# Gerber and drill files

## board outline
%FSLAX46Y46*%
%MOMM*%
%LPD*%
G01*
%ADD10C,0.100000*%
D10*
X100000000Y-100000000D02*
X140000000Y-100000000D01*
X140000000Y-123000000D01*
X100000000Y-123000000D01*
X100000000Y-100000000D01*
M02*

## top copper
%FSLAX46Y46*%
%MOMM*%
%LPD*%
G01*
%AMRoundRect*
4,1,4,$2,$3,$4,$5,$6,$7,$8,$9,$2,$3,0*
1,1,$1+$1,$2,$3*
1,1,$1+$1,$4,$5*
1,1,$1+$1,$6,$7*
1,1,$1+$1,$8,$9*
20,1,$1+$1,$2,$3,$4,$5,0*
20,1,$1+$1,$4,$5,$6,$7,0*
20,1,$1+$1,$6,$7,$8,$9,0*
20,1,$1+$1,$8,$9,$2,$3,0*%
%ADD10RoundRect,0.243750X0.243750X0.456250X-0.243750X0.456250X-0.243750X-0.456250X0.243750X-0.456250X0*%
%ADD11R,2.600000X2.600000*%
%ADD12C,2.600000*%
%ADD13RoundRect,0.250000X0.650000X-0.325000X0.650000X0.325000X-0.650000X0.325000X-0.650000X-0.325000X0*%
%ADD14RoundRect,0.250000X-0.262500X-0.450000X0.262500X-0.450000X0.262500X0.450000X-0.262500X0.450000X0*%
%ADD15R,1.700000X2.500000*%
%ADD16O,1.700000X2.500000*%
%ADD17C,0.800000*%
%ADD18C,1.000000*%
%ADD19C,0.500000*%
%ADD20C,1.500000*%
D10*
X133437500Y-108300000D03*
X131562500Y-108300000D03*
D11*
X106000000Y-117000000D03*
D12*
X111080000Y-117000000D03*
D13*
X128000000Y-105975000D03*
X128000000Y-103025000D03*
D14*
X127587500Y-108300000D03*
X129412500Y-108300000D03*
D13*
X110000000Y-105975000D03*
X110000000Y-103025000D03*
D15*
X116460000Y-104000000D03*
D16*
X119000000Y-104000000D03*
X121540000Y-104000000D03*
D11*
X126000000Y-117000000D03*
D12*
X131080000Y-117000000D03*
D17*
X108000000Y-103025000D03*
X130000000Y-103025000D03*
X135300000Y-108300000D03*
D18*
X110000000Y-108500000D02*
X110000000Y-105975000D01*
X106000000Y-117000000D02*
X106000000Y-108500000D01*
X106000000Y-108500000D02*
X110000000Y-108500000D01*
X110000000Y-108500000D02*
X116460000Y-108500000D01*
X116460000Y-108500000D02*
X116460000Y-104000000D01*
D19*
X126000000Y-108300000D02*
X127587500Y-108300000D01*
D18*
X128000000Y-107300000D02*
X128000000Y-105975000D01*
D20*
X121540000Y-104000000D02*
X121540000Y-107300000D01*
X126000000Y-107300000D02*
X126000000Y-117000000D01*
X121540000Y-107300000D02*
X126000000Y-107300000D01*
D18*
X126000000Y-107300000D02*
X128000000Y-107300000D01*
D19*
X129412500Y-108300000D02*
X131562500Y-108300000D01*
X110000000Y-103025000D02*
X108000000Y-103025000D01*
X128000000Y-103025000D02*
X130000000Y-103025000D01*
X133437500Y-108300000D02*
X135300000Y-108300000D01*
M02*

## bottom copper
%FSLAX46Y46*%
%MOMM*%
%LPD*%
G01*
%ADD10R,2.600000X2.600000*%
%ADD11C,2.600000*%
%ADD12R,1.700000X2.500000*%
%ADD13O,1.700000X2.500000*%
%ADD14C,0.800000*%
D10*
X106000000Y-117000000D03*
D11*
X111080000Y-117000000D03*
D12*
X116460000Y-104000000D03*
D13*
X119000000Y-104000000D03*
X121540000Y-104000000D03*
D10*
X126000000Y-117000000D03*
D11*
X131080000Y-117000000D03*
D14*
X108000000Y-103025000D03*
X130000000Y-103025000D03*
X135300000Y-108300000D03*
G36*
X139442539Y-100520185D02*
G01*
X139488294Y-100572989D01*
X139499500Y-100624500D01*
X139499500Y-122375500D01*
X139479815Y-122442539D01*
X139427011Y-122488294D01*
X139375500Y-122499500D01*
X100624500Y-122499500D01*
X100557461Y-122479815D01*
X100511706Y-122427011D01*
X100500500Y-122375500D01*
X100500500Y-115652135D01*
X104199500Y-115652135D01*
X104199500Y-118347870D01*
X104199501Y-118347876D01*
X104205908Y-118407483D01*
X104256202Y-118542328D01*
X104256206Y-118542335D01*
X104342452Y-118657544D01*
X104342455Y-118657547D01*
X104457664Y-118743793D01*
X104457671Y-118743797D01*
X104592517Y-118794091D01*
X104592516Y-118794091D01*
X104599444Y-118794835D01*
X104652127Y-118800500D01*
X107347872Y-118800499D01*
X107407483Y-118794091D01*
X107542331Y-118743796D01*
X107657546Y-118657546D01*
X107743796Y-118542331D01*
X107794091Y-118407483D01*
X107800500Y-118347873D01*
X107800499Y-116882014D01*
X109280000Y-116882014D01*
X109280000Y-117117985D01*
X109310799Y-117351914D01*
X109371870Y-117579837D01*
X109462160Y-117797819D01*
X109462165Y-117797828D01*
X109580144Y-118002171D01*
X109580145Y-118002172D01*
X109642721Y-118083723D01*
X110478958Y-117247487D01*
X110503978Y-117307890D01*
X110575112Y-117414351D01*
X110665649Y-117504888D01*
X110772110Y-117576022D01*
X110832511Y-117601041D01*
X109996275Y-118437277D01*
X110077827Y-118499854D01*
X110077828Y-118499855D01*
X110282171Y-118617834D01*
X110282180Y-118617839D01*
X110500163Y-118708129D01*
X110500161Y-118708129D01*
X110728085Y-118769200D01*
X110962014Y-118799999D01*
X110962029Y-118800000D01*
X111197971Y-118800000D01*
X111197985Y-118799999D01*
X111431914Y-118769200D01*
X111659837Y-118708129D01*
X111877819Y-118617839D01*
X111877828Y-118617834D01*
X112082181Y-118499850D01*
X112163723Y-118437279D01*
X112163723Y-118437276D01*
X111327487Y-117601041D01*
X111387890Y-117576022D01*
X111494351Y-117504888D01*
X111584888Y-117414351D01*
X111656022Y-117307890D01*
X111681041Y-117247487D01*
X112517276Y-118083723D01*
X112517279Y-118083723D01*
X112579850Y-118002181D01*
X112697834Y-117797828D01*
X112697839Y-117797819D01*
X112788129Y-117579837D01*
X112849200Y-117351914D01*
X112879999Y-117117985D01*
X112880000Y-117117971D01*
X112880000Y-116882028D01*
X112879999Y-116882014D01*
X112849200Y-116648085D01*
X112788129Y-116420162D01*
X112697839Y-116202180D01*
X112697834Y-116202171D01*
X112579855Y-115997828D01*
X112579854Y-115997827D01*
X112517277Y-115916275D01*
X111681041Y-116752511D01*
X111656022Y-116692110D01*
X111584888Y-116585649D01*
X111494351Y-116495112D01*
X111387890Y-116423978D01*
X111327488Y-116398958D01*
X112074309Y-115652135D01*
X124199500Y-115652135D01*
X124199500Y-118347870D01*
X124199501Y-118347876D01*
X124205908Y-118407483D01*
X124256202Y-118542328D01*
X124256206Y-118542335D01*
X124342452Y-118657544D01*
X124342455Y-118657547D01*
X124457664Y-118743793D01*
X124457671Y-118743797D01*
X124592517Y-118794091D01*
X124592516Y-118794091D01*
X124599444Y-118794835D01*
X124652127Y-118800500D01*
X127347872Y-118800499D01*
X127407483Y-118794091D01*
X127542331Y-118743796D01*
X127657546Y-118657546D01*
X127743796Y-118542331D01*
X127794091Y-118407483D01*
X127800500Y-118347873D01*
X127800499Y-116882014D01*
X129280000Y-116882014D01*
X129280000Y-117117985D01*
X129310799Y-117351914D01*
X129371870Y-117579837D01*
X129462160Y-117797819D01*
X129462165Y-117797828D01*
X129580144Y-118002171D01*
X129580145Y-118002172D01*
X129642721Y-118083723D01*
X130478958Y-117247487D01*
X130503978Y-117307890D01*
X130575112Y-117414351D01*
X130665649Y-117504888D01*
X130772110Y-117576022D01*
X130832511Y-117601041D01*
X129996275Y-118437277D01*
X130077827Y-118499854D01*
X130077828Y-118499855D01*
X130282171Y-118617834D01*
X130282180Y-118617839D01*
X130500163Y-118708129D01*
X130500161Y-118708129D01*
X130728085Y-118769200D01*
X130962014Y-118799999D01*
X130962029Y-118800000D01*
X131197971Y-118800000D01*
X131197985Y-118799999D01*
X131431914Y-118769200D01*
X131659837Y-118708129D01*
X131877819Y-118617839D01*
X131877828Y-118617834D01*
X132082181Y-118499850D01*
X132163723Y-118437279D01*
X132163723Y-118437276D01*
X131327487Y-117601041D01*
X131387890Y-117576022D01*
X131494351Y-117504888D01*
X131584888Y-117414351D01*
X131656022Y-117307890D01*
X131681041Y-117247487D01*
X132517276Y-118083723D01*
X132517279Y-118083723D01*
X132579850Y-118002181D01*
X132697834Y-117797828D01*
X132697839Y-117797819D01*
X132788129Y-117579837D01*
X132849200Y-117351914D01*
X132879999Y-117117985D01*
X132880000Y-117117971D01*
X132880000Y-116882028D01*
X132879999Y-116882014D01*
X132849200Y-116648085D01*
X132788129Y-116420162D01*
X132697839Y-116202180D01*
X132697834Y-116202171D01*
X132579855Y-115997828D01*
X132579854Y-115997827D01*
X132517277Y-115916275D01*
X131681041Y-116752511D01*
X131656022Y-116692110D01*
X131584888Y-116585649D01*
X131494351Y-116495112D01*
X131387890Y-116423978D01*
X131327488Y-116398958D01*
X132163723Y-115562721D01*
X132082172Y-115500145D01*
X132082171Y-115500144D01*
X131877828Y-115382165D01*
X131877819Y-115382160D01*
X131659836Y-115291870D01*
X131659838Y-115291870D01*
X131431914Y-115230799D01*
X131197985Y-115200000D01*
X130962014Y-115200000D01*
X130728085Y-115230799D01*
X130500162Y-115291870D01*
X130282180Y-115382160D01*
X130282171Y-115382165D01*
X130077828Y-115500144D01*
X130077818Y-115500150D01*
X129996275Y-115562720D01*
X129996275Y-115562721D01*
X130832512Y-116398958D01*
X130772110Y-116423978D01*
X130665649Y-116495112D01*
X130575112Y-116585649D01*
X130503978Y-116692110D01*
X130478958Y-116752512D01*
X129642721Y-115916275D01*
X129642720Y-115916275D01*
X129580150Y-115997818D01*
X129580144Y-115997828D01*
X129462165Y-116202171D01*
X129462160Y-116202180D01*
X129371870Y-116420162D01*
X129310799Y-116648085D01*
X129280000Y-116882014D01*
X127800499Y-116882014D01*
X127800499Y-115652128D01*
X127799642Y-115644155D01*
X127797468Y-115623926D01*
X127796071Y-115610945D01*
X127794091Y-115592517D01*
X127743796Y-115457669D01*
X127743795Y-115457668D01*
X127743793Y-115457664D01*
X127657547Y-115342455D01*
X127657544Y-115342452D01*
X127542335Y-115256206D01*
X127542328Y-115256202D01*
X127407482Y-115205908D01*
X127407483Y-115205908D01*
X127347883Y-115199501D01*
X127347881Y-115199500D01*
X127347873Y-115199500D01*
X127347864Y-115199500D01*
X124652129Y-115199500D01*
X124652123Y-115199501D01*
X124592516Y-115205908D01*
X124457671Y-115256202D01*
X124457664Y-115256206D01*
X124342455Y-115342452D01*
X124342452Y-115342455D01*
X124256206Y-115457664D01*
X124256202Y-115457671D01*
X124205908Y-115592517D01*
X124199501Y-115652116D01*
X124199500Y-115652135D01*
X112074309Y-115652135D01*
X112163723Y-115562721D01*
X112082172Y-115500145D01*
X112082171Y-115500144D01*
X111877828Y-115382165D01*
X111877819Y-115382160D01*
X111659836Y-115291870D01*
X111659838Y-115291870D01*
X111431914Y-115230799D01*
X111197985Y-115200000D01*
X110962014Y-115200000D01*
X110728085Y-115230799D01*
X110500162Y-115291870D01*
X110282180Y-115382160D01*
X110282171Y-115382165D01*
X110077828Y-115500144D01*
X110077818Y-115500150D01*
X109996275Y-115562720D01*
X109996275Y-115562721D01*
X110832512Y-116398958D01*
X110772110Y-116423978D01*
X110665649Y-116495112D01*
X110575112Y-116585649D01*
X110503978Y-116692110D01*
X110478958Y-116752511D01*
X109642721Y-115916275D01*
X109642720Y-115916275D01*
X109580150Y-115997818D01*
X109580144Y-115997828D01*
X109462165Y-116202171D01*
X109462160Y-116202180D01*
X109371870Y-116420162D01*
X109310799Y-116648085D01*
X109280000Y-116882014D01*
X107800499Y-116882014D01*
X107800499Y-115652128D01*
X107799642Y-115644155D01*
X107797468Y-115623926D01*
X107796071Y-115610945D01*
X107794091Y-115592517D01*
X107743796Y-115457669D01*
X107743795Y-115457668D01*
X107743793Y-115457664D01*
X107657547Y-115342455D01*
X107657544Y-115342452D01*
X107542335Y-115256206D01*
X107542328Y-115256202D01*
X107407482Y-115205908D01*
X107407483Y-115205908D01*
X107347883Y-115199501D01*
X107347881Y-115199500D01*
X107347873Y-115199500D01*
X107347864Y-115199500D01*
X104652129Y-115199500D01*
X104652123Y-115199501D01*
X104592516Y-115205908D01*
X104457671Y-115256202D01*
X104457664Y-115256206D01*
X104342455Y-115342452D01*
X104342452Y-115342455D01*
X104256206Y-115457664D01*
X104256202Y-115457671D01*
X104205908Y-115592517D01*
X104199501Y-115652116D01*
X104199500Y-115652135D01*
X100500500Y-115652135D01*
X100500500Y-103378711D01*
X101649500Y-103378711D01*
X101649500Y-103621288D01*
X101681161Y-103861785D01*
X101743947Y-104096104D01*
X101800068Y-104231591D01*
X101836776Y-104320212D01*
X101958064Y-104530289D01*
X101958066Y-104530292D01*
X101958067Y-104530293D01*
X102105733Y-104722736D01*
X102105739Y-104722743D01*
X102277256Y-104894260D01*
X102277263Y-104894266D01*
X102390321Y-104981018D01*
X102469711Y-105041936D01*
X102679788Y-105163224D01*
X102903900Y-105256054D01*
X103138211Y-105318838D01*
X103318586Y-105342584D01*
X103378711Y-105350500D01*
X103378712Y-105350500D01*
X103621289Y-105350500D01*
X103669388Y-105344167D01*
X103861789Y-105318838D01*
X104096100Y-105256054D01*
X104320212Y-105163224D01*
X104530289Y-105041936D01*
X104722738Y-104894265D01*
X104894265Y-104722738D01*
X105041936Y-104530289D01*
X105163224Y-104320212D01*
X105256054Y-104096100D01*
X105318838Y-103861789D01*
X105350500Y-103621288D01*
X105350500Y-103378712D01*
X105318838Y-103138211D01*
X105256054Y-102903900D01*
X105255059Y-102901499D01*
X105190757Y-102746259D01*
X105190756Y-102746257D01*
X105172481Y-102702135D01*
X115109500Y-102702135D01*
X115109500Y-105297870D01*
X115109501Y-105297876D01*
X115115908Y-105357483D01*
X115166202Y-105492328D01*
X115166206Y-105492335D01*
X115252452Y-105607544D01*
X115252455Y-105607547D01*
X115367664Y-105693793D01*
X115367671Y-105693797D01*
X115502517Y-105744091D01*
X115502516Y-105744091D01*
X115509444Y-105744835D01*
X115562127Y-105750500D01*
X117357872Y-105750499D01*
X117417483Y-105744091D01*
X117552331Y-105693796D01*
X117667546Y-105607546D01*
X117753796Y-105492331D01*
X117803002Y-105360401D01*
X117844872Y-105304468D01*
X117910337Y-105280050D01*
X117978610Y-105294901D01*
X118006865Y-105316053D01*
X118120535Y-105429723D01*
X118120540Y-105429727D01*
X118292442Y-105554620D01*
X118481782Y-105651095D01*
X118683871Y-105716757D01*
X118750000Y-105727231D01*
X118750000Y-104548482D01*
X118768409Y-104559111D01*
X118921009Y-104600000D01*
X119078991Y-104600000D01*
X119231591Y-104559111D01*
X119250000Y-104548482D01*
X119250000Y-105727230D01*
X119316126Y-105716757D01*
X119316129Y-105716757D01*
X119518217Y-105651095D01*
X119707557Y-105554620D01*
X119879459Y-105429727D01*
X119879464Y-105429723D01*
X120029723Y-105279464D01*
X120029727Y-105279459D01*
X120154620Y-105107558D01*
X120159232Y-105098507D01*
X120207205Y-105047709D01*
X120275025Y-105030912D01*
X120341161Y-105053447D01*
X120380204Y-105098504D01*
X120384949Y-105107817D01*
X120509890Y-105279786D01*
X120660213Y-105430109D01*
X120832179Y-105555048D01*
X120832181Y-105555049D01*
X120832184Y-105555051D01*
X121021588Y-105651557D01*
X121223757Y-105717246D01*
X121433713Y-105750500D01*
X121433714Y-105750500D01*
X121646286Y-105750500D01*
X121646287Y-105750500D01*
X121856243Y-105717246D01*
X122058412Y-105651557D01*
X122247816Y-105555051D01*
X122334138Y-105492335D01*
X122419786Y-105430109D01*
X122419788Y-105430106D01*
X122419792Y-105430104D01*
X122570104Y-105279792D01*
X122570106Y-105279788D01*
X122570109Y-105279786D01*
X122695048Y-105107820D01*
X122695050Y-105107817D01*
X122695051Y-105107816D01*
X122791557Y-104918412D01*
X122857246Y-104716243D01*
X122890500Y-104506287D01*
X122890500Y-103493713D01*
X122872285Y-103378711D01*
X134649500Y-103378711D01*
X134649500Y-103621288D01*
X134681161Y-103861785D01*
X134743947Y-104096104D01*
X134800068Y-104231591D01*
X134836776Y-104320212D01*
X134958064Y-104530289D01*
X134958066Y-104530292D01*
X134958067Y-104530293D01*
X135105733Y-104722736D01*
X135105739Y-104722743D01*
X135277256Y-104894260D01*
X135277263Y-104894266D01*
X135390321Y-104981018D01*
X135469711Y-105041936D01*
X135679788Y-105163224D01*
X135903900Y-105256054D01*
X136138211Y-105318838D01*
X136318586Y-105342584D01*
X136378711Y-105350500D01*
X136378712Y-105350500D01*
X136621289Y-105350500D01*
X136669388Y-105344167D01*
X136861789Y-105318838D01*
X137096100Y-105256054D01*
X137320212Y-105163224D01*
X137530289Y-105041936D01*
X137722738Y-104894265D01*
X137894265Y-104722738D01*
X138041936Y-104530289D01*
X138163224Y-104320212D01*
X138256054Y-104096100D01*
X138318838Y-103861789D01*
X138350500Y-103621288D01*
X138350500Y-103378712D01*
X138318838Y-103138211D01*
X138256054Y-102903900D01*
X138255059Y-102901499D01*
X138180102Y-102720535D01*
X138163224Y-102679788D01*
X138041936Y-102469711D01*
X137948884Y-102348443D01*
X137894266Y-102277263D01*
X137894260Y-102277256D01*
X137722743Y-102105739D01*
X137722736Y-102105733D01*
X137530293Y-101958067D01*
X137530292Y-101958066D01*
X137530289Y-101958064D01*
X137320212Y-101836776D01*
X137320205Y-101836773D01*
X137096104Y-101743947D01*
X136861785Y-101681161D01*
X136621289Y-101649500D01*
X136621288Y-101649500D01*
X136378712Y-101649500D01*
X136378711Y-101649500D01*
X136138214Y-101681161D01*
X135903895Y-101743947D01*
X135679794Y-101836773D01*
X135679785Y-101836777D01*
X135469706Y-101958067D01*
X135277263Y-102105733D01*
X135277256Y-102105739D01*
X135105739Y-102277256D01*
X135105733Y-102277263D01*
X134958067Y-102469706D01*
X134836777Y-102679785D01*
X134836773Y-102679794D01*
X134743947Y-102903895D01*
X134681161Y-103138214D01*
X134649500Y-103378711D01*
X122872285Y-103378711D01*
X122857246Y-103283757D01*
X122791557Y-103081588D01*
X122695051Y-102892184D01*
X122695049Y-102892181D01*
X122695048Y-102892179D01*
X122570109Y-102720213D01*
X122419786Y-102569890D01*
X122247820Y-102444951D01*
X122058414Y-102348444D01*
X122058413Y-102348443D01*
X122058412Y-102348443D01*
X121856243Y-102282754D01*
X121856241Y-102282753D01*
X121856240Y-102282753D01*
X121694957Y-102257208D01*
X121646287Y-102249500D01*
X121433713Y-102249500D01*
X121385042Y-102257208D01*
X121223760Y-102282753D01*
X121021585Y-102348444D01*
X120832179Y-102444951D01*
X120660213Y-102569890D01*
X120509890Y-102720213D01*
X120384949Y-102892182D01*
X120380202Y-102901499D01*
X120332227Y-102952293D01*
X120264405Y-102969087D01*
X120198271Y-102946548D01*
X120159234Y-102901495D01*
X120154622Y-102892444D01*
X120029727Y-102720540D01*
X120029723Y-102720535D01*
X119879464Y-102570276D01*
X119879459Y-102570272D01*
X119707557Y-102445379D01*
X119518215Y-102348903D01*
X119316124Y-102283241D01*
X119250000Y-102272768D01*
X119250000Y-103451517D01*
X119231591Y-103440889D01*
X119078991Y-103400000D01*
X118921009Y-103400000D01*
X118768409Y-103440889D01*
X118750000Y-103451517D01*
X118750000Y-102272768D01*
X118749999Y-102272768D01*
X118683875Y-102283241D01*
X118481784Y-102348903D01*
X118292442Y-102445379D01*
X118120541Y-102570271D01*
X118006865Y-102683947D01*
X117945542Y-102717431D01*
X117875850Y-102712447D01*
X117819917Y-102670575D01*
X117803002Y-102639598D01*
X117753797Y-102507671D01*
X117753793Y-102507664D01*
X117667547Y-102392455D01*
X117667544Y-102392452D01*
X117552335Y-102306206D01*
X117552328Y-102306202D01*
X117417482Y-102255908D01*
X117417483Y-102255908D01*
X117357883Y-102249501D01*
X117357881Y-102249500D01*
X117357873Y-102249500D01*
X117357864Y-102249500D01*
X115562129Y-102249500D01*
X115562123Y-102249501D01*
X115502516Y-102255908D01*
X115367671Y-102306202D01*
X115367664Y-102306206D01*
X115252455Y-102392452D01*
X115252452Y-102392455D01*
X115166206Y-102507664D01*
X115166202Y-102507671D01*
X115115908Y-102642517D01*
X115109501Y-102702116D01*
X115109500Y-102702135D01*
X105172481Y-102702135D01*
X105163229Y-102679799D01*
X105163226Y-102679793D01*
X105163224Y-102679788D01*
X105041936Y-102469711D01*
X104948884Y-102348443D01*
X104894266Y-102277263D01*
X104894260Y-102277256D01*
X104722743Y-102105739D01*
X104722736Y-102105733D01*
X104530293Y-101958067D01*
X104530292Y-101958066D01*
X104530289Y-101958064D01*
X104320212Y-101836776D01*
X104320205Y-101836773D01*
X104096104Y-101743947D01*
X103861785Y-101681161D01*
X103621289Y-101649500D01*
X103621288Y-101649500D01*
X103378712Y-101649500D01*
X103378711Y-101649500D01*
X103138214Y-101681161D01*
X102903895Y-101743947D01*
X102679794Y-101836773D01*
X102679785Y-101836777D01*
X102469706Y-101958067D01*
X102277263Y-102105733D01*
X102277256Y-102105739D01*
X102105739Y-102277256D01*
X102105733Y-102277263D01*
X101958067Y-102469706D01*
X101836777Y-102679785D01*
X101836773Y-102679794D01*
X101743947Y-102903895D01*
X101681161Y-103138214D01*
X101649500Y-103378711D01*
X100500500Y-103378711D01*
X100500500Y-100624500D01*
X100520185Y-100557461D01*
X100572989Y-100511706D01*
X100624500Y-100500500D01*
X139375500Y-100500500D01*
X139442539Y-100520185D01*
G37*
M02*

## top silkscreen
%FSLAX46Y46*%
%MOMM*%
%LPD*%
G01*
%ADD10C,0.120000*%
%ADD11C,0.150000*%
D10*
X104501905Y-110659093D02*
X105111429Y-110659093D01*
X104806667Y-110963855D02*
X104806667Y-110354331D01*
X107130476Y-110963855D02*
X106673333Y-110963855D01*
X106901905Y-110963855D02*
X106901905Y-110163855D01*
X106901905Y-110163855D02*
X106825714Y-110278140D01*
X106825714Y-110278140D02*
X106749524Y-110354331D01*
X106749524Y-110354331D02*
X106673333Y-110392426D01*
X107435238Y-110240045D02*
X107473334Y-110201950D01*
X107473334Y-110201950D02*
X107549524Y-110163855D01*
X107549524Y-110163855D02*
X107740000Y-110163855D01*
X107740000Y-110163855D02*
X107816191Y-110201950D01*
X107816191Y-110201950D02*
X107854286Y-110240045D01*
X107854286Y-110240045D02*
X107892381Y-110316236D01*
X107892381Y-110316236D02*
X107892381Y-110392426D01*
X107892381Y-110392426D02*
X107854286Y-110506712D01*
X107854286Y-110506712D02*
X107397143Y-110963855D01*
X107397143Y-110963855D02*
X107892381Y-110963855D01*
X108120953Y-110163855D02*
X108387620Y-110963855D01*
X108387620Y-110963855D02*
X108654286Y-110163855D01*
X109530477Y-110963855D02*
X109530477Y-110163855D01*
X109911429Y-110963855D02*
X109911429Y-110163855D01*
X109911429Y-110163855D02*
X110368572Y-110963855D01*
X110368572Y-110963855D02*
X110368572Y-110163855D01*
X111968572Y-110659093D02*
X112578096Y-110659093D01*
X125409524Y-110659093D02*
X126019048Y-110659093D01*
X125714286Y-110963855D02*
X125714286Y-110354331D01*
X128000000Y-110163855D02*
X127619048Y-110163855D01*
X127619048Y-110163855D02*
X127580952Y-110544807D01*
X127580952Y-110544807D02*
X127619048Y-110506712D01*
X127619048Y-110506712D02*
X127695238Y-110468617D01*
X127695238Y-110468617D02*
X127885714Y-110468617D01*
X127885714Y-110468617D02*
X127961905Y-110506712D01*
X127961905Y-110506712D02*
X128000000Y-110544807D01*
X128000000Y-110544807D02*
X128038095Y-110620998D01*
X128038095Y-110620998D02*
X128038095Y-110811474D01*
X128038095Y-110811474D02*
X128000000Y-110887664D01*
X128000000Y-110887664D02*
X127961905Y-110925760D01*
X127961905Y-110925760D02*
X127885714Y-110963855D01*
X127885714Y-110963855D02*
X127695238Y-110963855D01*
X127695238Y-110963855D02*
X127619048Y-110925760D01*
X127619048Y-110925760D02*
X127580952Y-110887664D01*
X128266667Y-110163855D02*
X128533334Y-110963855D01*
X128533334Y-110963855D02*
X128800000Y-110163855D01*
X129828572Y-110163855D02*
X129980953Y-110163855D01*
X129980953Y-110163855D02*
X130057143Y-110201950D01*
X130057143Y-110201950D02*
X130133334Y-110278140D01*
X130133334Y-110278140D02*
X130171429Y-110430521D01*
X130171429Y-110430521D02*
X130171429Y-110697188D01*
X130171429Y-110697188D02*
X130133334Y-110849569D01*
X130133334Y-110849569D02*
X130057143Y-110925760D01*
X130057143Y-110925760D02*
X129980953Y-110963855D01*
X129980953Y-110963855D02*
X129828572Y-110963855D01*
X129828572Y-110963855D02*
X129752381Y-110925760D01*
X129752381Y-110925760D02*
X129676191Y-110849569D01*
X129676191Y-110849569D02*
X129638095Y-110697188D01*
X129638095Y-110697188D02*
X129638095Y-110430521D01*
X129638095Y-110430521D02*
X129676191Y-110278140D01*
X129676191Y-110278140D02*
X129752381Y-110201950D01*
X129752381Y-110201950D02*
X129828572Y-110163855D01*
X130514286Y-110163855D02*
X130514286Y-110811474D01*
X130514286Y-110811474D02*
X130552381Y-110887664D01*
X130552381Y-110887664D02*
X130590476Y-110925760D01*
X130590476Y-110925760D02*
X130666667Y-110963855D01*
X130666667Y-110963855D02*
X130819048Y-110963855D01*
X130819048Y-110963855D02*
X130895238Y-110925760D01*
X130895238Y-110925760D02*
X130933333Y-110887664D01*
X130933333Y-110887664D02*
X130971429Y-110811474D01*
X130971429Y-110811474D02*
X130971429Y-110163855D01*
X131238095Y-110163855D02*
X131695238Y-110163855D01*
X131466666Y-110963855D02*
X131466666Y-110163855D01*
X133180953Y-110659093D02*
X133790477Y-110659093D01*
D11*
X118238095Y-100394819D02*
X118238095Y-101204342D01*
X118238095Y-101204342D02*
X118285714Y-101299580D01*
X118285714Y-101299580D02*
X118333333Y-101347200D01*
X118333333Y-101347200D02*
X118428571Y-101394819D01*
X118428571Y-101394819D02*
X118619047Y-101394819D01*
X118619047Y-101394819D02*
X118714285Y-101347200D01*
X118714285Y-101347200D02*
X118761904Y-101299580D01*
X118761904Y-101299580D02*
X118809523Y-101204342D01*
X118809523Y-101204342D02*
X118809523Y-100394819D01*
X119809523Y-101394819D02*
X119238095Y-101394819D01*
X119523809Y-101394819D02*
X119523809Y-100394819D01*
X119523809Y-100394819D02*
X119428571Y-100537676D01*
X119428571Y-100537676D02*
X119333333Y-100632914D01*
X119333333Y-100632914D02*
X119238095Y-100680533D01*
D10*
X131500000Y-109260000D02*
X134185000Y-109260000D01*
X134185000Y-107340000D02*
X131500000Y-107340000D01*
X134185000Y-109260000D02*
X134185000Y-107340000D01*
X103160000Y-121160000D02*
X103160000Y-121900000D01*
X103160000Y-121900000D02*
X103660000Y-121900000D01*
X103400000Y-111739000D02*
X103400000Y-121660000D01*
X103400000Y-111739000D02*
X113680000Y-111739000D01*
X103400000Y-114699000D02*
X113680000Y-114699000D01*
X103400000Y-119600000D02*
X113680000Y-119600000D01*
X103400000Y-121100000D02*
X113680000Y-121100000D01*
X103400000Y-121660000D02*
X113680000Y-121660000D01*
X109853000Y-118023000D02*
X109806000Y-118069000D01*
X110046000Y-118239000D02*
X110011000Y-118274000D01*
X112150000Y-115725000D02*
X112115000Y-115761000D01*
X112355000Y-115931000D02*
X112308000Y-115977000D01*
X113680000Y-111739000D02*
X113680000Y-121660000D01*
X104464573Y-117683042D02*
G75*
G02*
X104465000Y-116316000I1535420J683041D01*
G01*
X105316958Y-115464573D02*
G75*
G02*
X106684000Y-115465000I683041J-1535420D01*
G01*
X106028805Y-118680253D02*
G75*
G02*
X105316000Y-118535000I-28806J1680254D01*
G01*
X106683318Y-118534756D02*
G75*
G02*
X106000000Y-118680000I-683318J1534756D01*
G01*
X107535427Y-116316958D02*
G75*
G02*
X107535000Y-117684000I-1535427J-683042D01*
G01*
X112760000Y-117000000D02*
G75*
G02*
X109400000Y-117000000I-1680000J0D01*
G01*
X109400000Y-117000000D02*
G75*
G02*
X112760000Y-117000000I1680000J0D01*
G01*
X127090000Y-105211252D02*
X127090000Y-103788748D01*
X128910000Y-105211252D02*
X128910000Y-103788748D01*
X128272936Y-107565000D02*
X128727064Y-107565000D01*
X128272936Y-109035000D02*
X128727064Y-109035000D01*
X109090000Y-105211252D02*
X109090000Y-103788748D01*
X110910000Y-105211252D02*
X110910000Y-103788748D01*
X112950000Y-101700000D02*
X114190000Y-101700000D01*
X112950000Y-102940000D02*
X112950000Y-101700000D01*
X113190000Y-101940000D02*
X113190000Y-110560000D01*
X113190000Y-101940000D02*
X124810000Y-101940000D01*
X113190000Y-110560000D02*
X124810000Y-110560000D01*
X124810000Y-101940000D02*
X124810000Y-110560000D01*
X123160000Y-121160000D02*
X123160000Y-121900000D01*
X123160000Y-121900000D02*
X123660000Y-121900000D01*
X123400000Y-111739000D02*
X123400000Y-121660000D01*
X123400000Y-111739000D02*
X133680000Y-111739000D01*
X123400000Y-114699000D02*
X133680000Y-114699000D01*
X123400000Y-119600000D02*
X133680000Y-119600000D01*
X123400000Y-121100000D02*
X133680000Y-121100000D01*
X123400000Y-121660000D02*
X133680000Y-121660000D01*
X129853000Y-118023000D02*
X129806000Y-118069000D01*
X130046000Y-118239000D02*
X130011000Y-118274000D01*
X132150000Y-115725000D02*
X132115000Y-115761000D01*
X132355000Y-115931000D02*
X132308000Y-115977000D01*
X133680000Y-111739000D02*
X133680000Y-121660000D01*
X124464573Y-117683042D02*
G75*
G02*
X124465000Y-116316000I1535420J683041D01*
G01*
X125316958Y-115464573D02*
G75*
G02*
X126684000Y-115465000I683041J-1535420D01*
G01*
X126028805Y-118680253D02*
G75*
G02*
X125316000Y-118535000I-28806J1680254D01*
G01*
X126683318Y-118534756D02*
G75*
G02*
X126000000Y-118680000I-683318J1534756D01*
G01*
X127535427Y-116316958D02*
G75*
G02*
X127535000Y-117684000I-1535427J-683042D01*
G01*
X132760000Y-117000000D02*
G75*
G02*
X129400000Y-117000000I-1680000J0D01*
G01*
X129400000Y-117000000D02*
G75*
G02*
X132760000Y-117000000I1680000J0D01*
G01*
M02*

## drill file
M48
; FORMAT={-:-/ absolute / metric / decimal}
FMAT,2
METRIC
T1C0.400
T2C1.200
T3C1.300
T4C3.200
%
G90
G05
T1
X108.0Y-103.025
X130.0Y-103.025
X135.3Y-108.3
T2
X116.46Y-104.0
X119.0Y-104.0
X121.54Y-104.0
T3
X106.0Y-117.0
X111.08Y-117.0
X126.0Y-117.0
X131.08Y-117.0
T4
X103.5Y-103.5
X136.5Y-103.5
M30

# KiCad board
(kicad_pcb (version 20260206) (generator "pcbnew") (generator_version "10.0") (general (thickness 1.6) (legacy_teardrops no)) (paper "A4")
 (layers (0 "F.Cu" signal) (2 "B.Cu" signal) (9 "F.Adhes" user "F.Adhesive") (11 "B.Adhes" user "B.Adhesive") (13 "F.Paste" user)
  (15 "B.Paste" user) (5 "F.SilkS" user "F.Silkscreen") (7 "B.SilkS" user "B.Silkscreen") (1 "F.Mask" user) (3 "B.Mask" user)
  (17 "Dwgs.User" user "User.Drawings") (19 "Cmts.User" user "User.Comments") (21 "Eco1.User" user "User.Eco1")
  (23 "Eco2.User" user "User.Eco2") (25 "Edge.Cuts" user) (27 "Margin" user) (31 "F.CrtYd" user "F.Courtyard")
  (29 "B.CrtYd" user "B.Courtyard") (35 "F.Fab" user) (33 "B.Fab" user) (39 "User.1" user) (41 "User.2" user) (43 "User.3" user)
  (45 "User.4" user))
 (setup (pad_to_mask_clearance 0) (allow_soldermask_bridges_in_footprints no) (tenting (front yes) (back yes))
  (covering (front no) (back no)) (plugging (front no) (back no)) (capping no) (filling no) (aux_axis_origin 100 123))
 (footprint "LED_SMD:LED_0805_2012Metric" (layer "F.Cu") (at 132.5 108.3 180)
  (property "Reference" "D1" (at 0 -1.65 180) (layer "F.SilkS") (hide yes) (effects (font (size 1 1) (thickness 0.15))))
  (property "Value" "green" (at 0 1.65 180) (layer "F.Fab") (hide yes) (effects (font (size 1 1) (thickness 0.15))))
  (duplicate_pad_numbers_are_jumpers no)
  (fp_line (start 1 -0.96) (end -1.685 -0.96) (stroke (width 0.12) (type solid)) (layer "F.SilkS"))
  (fp_line (start -1.685 0.96) (end 1 0.96) (stroke (width 0.12) (type solid)) (layer "F.SilkS"))
  (fp_line (start -1.685 -0.96) (end -1.685 0.96) (stroke (width 0.12) (type solid)) (layer "F.SilkS"))
  (pad "1" smd roundrect (at -0.9375 0 180) (size 0.975 1.4) (layers "F.Cu" "F.Mask" "F.Paste") (roundrect_rratio 0.25) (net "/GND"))
  (pad "2" smd roundrect (at 0.9375 0 180) (size 0.975 1.4) (layers "F.Cu" "F.Mask" "F.Paste") (roundrect_rratio 0.25) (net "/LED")))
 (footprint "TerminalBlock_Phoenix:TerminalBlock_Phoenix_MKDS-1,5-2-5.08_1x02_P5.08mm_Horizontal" (layer "F.Cu") (at 106 117)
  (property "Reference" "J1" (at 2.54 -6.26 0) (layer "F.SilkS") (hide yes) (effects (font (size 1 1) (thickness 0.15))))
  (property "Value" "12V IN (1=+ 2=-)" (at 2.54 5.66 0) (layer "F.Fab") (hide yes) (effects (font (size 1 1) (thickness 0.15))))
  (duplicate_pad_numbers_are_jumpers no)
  (fp_line (start -2.84 4.16) (end -2.84 4.9) (stroke (width 0.12) (type solid)) (layer "F.SilkS"))
  (fp_line (start -2.84 4.9) (end -2.34 4.9) (stroke (width 0.12) (type solid)) (layer "F.SilkS"))
  (fp_line (start -2.6 -5.261) (end -2.6 4.66) (stroke (width 0.12) (type solid)) (layer "F.SilkS"))
  (fp_line (start -2.6 -5.261) (end 7.68 -5.261) (stroke (width 0.12) (type solid)) (layer "F.SilkS"))
  (fp_line (start -2.6 -2.301) (end 7.68 -2.301) (stroke (width 0.12) (type solid)) (layer "F.SilkS"))
  (fp_line (start -2.6 2.6) (end 7.68 2.6) (stroke (width 0.12) (type solid)) (layer "F.SilkS"))
  (fp_line (start -2.6 4.1) (end 7.68 4.1) (stroke (width 0.12) (type solid)) (layer "F.SilkS"))
  (fp_line (start -2.6 4.66) (end 7.68 4.66) (stroke (width 0.12) (type solid)) (layer "F.SilkS"))
  (fp_line (start 3.853 1.023) (end 3.806 1.069) (stroke (width 0.12) (type solid)) (layer "F.SilkS"))
  (fp_line (start 4.046 1.239) (end 4.011 1.274) (stroke (width 0.12) (type solid)) (layer "F.SilkS"))
  (fp_line (start 6.15 -1.275) (end 6.115 -1.239) (stroke (width 0.12) (type solid)) (layer "F.SilkS"))
  (fp_line (start 6.355 -1.069) (end 6.308 -1.023) (stroke (width 0.12) (type solid)) (layer "F.SilkS"))
  (fp_line (start 7.68 -5.261) (end 7.68 4.66) (stroke (width 0.12) (type solid)) (layer "F.SilkS"))
  (fp_arc (start -1.535427 0.683042) (mid -1.680501 -0.000524) (end -1.535 -0.684) (stroke (width 0.12) (type solid)) (layer "F.SilkS"))
  (fp_arc (start -0.683042 -1.535427) (mid 0.000524 -1.680501) (end 0.684 -1.535) (stroke (width 0.12) (type solid)) (layer "F.SilkS"))
  (fp_arc (start 0.028805 1.680253) (mid -0.335551 1.646659) (end -0.684 1.535) (stroke (width 0.12) (type solid)) (layer "F.SilkS"))
  (fp_arc (start 0.683318 1.534756) (mid 0.349292 1.643288) (end 0 1.68) (stroke (width 0.12) (type solid)) (layer "F.SilkS"))
  (fp_arc (start 1.535427 -0.683042) (mid 1.680501 0.000524) (end 1.535 0.684) (stroke (width 0.12) (type solid)) (layer "F.SilkS"))
  (fp_circle (center 5.08 0) (end 6.76 0) (stroke (width 0.12) (type solid)) (fill no) (layer "F.SilkS"))
  (pad "1" thru_hole rect (at 0 0) (size 2.6 2.6) (drill 1.3) (layers "*.Cu" "*.Mask") (remove_unused_layers no) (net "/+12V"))
  (pad "2" thru_hole circle (at 5.08 0) (size 2.6 2.6) (drill 1.3) (layers "*.Cu" "*.Mask") (remove_unused_layers no) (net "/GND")))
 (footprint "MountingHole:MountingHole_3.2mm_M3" (layer "F.Cu") (at 103.5 103.5)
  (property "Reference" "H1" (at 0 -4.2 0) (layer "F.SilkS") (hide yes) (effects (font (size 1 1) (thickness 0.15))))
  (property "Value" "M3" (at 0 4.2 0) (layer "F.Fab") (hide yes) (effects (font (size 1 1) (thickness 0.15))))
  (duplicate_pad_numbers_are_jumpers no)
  (pad "" np_thru_hole circle (at 0 0) (size 3.2 3.2) (drill 3.2) (layers "*.Cu" "*.Mask")))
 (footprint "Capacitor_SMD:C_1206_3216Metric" (layer "F.Cu") (at 128 104.5 90)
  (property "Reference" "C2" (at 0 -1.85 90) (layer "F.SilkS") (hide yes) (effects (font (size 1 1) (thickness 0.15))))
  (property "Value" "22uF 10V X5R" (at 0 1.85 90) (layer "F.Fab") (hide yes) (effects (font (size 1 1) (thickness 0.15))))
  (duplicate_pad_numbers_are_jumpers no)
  (fp_line (start -0.711252 -0.91) (end 0.711252 -0.91) (stroke (width 0.12) (type solid)) (layer "F.SilkS"))
  (fp_line (start -0.711252 0.91) (end 0.711252 0.91) (stroke (width 0.12) (type solid)) (layer "F.SilkS"))
  (pad "1" smd roundrect (at -1.475 0 90) (size 1.15 1.8) (layers "F.Cu" "F.Mask" "F.Paste") (roundrect_rratio 0.217391) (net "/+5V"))
  (pad "2" smd roundrect (at 1.475 0 90) (size 1.15 1.8) (layers "F.Cu" "F.Mask" "F.Paste") (roundrect_rratio 0.217391) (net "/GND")))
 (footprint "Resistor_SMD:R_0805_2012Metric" (layer "F.Cu") (at 128.5 108.3)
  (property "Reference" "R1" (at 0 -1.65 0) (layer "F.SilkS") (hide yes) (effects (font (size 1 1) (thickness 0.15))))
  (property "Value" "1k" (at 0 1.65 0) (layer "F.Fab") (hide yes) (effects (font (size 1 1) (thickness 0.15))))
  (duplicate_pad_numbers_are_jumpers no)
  (fp_line (start -0.227064 -0.735) (end 0.227064 -0.735) (stroke (width 0.12) (type solid)) (layer "F.SilkS"))
  (fp_line (start -0.227064 0.735) (end 0.227064 0.735) (stroke (width 0.12) (type solid)) (layer "F.SilkS"))
  (pad "1" smd roundrect (at -0.9125 0) (size 1.025 1.4) (layers "F.Cu" "F.Mask" "F.Paste") (roundrect_rratio 0.243902) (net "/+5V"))
  (pad "2" smd roundrect (at 0.9125 0) (size 1.025 1.4) (layers "F.Cu" "F.Mask" "F.Paste") (roundrect_rratio 0.243902) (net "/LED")))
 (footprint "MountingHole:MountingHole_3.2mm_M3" (layer "F.Cu") (at 136.5 103.5)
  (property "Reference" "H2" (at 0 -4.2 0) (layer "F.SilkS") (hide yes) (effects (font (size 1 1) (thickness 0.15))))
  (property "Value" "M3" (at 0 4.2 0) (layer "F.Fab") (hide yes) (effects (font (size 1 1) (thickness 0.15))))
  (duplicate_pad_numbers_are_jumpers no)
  (pad "" np_thru_hole circle (at 0 0) (size 3.2 3.2) (drill 3.2) (layers "*.Cu" "*.Mask")))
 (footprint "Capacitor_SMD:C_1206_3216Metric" (layer "F.Cu") (at 110 104.5 90)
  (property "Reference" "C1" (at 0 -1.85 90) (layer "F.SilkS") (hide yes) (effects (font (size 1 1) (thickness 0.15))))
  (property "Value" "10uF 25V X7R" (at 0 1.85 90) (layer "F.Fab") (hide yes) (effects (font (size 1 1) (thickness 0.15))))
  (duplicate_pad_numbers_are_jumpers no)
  (fp_line (start -0.711252 -0.91) (end 0.711252 -0.91) (stroke (width 0.12) (type solid)) (layer "F.SilkS"))
  (fp_line (start -0.711252 0.91) (end 0.711252 0.91) (stroke (width 0.12) (type solid)) (layer "F.SilkS"))
  (pad "1" smd roundrect (at -1.475 0 90) (size 1.15 1.8) (layers "F.Cu" "F.Mask" "F.Paste") (roundrect_rratio 0.217391) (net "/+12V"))
  (pad "2" smd roundrect (at 1.475 0 90) (size 1.15 1.8) (layers "F.Cu" "F.Mask" "F.Paste") (roundrect_rratio 0.217391) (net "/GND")))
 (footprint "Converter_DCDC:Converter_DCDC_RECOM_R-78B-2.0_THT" (layer "F.Cu") (at 116.46 104)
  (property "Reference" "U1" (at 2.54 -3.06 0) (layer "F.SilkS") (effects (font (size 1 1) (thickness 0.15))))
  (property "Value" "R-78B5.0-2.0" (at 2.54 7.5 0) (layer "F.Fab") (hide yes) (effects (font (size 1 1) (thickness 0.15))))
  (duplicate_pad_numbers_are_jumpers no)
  (fp_line (start -3.51 -2.3) (end -2.27 -2.3) (stroke (width 0.12) (type solid)) (layer "F.SilkS"))
  (fp_line (start -3.51 -1.06) (end -3.51 -2.3) (stroke (width 0.12) (type solid)) (layer "F.SilkS"))
  (fp_line (start -3.27 -2.06) (end -3.27 6.56) (stroke (width 0.12) (type solid)) (layer "F.SilkS"))
  (fp_line (start -3.27 -2.06) (end 8.35 -2.06) (stroke (width 0.12) (type solid)) (layer "F.SilkS"))
  (fp_line (start -3.27 6.56) (end 8.35 6.56) (stroke (width 0.12) (type solid)) (layer "F.SilkS"))
  (fp_line (start 8.35 -2.06) (end 8.35 6.56) (stroke (width 0.12) (type solid)) (layer "F.SilkS"))
  (pad "1" thru_hole rect (at 0 0) (size 1.7 2.5) (drill 1.2) (layers "*.Cu" "*.Mask") (remove_unused_layers no) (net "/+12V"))
  (pad "2" thru_hole oval (at 2.54 0) (size 1.7 2.5) (drill 1.2) (layers "*.Cu" "*.Mask") (remove_unused_layers no) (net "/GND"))
  (pad "3" thru_hole oval (at 5.08 0) (size 1.7 2.5) (drill 1.2) (layers "*.Cu" "*.Mask") (remove_unused_layers no) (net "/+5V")))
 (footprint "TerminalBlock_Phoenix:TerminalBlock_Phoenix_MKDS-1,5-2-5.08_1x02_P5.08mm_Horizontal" (layer "F.Cu") (at 126 117)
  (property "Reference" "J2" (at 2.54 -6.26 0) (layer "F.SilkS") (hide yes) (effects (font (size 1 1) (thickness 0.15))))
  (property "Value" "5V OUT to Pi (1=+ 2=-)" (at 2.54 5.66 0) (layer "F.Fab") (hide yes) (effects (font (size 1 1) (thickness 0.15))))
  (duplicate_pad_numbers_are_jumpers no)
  (fp_line (start -2.84 4.16) (end -2.84 4.9) (stroke (width 0.12) (type solid)) (layer "F.SilkS"))
  (fp_line (start -2.84 4.9) (end -2.34 4.9) (stroke (width 0.12) (type solid)) (layer "F.SilkS"))
  (fp_line (start -2.6 -5.261) (end -2.6 4.66) (stroke (width 0.12) (type solid)) (layer "F.SilkS"))
  (fp_line (start -2.6 -5.261) (end 7.68 -5.261) (stroke (width 0.12) (type solid)) (layer "F.SilkS"))
  (fp_line (start -2.6 -2.301) (end 7.68 -2.301) (stroke (width 0.12) (type solid)) (layer "F.SilkS"))
  (fp_line (start -2.6 2.6) (end 7.68 2.6) (stroke (width 0.12) (type solid)) (layer "F.SilkS"))
  (fp_line (start -2.6 4.1) (end 7.68 4.1) (stroke (width 0.12) (type solid)) (layer "F.SilkS"))
  (fp_line (start -2.6 4.66) (end 7.68 4.66) (stroke (width 0.12) (type solid)) (layer "F.SilkS"))
  (fp_line (start 3.853 1.023) (end 3.806 1.069) (stroke (width 0.12) (type solid)) (layer "F.SilkS"))
  (fp_line (start 4.046 1.239) (end 4.011 1.274) (stroke (width 0.12) (type solid)) (layer "F.SilkS"))
  (fp_line (start 6.15 -1.275) (end 6.115 -1.239) (stroke (width 0.12) (type solid)) (layer "F.SilkS"))
  (fp_line (start 6.355 -1.069) (end 6.308 -1.023) (stroke (width 0.12) (type solid)) (layer "F.SilkS"))
  (fp_line (start 7.68 -5.261) (end 7.68 4.66) (stroke (width 0.12) (type solid)) (layer "F.SilkS"))
  (fp_arc (start -1.535427 0.683042) (mid -1.680501 -0.000524) (end -1.535 -0.684) (stroke (width 0.12) (type solid)) (layer "F.SilkS"))
  (fp_arc (start -0.683042 -1.535427) (mid 0.000524 -1.680501) (end 0.684 -1.535) (stroke (width 0.12) (type solid)) (layer "F.SilkS"))
  (fp_arc (start 0.028805 1.680253) (mid -0.335551 1.646659) (end -0.684 1.535) (stroke (width 0.12) (type solid)) (layer "F.SilkS"))
  (fp_arc (start 0.683318 1.534756) (mid 0.349292 1.643288) (end 0 1.68) (stroke (width 0.12) (type solid)) (layer "F.SilkS"))
  (fp_arc (start 1.535427 -0.683042) (mid 1.680501 0.000524) (end 1.535 0.684) (stroke (width 0.12) (type solid)) (layer "F.SilkS"))
  (fp_circle (center 5.08 0) (end 6.76 0) (stroke (width 0.12) (type solid)) (fill no) (layer "F.SilkS"))
  (pad "1" thru_hole rect (at 0 0) (size 2.6 2.6) (drill 1.3) (layers "*.Cu" "*.Mask") (remove_unused_layers no) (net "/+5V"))
  (pad "2" thru_hole circle (at 5.08 0) (size 2.6 2.6) (drill 1.3) (layers "*.Cu" "*.Mask") (remove_unused_layers no) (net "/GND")))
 (gr_rect (start 100 100) (end 140 123) (stroke (width 0.1) (type default)) (fill no) (layer "Edge.Cuts"))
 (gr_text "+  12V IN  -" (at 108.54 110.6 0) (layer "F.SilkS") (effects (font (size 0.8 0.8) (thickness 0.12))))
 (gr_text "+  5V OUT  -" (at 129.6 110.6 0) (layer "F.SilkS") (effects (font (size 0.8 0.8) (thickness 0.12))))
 (segment (start 110 108.5) (end 110 105.975) (width 1) (layer "F.Cu") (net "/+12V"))
 (segment (start 106 117) (end 106 108.5) (width 1) (layer "F.Cu") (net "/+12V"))
 (segment (start 106 108.5) (end 110 108.5) (width 1) (layer "F.Cu") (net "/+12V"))
 (segment (start 110 108.5) (end 116.46 108.5) (width 1) (layer "F.Cu") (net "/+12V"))
 (segment (start 116.46 108.5) (end 116.46 104) (width 1) (layer "F.Cu") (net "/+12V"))
 (segment (start 126 108.3) (end 127.5875 108.3) (width 0.5) (layer "F.Cu") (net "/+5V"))
 (segment (start 128 107.3) (end 128 105.975) (width 1) (layer "F.Cu") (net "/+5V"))
 (segment (start 121.54 104) (end 121.54 107.3) (width 1.5) (layer "F.Cu") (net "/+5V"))
 (segment (start 126 107.3) (end 126 117) (width 1.5) (layer "F.Cu") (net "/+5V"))
 (segment (start 121.54 107.3) (end 126 107.3) (width 1.5) (layer "F.Cu") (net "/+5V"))
 (segment (start 126 107.3) (end 128 107.3) (width 1) (layer "F.Cu") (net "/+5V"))
 (segment (start 129.4125 108.3) (end 131.5625 108.3) (width 0.5) (layer "F.Cu") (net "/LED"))
 (segment (start 110 103.025) (end 108 103.025) (width 0.5) (layer "F.Cu") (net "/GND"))
 (segment (start 128 103.025) (end 130 103.025) (width 0.5) (layer "F.Cu") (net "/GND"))
 (segment (start 133.4375 108.3) (end 135.3 108.3) (width 0.5) (layer "F.Cu") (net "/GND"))
 (via (at 108 103.025) (size 0.8) (drill 0.4) (layers "F.Cu" "B.Cu") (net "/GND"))
 (via (at 130 103.025) (size 0.8) (drill 0.4) (layers "F.Cu" "B.Cu") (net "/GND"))
 (via (at 135.3 108.3) (size 0.8) (drill 0.4) (layers "F.Cu" "B.Cu") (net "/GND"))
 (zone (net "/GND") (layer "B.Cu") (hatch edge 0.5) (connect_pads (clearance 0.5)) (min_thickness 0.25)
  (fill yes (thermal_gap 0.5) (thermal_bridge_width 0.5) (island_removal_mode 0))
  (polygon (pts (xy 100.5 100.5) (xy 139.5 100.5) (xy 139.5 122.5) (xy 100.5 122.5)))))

